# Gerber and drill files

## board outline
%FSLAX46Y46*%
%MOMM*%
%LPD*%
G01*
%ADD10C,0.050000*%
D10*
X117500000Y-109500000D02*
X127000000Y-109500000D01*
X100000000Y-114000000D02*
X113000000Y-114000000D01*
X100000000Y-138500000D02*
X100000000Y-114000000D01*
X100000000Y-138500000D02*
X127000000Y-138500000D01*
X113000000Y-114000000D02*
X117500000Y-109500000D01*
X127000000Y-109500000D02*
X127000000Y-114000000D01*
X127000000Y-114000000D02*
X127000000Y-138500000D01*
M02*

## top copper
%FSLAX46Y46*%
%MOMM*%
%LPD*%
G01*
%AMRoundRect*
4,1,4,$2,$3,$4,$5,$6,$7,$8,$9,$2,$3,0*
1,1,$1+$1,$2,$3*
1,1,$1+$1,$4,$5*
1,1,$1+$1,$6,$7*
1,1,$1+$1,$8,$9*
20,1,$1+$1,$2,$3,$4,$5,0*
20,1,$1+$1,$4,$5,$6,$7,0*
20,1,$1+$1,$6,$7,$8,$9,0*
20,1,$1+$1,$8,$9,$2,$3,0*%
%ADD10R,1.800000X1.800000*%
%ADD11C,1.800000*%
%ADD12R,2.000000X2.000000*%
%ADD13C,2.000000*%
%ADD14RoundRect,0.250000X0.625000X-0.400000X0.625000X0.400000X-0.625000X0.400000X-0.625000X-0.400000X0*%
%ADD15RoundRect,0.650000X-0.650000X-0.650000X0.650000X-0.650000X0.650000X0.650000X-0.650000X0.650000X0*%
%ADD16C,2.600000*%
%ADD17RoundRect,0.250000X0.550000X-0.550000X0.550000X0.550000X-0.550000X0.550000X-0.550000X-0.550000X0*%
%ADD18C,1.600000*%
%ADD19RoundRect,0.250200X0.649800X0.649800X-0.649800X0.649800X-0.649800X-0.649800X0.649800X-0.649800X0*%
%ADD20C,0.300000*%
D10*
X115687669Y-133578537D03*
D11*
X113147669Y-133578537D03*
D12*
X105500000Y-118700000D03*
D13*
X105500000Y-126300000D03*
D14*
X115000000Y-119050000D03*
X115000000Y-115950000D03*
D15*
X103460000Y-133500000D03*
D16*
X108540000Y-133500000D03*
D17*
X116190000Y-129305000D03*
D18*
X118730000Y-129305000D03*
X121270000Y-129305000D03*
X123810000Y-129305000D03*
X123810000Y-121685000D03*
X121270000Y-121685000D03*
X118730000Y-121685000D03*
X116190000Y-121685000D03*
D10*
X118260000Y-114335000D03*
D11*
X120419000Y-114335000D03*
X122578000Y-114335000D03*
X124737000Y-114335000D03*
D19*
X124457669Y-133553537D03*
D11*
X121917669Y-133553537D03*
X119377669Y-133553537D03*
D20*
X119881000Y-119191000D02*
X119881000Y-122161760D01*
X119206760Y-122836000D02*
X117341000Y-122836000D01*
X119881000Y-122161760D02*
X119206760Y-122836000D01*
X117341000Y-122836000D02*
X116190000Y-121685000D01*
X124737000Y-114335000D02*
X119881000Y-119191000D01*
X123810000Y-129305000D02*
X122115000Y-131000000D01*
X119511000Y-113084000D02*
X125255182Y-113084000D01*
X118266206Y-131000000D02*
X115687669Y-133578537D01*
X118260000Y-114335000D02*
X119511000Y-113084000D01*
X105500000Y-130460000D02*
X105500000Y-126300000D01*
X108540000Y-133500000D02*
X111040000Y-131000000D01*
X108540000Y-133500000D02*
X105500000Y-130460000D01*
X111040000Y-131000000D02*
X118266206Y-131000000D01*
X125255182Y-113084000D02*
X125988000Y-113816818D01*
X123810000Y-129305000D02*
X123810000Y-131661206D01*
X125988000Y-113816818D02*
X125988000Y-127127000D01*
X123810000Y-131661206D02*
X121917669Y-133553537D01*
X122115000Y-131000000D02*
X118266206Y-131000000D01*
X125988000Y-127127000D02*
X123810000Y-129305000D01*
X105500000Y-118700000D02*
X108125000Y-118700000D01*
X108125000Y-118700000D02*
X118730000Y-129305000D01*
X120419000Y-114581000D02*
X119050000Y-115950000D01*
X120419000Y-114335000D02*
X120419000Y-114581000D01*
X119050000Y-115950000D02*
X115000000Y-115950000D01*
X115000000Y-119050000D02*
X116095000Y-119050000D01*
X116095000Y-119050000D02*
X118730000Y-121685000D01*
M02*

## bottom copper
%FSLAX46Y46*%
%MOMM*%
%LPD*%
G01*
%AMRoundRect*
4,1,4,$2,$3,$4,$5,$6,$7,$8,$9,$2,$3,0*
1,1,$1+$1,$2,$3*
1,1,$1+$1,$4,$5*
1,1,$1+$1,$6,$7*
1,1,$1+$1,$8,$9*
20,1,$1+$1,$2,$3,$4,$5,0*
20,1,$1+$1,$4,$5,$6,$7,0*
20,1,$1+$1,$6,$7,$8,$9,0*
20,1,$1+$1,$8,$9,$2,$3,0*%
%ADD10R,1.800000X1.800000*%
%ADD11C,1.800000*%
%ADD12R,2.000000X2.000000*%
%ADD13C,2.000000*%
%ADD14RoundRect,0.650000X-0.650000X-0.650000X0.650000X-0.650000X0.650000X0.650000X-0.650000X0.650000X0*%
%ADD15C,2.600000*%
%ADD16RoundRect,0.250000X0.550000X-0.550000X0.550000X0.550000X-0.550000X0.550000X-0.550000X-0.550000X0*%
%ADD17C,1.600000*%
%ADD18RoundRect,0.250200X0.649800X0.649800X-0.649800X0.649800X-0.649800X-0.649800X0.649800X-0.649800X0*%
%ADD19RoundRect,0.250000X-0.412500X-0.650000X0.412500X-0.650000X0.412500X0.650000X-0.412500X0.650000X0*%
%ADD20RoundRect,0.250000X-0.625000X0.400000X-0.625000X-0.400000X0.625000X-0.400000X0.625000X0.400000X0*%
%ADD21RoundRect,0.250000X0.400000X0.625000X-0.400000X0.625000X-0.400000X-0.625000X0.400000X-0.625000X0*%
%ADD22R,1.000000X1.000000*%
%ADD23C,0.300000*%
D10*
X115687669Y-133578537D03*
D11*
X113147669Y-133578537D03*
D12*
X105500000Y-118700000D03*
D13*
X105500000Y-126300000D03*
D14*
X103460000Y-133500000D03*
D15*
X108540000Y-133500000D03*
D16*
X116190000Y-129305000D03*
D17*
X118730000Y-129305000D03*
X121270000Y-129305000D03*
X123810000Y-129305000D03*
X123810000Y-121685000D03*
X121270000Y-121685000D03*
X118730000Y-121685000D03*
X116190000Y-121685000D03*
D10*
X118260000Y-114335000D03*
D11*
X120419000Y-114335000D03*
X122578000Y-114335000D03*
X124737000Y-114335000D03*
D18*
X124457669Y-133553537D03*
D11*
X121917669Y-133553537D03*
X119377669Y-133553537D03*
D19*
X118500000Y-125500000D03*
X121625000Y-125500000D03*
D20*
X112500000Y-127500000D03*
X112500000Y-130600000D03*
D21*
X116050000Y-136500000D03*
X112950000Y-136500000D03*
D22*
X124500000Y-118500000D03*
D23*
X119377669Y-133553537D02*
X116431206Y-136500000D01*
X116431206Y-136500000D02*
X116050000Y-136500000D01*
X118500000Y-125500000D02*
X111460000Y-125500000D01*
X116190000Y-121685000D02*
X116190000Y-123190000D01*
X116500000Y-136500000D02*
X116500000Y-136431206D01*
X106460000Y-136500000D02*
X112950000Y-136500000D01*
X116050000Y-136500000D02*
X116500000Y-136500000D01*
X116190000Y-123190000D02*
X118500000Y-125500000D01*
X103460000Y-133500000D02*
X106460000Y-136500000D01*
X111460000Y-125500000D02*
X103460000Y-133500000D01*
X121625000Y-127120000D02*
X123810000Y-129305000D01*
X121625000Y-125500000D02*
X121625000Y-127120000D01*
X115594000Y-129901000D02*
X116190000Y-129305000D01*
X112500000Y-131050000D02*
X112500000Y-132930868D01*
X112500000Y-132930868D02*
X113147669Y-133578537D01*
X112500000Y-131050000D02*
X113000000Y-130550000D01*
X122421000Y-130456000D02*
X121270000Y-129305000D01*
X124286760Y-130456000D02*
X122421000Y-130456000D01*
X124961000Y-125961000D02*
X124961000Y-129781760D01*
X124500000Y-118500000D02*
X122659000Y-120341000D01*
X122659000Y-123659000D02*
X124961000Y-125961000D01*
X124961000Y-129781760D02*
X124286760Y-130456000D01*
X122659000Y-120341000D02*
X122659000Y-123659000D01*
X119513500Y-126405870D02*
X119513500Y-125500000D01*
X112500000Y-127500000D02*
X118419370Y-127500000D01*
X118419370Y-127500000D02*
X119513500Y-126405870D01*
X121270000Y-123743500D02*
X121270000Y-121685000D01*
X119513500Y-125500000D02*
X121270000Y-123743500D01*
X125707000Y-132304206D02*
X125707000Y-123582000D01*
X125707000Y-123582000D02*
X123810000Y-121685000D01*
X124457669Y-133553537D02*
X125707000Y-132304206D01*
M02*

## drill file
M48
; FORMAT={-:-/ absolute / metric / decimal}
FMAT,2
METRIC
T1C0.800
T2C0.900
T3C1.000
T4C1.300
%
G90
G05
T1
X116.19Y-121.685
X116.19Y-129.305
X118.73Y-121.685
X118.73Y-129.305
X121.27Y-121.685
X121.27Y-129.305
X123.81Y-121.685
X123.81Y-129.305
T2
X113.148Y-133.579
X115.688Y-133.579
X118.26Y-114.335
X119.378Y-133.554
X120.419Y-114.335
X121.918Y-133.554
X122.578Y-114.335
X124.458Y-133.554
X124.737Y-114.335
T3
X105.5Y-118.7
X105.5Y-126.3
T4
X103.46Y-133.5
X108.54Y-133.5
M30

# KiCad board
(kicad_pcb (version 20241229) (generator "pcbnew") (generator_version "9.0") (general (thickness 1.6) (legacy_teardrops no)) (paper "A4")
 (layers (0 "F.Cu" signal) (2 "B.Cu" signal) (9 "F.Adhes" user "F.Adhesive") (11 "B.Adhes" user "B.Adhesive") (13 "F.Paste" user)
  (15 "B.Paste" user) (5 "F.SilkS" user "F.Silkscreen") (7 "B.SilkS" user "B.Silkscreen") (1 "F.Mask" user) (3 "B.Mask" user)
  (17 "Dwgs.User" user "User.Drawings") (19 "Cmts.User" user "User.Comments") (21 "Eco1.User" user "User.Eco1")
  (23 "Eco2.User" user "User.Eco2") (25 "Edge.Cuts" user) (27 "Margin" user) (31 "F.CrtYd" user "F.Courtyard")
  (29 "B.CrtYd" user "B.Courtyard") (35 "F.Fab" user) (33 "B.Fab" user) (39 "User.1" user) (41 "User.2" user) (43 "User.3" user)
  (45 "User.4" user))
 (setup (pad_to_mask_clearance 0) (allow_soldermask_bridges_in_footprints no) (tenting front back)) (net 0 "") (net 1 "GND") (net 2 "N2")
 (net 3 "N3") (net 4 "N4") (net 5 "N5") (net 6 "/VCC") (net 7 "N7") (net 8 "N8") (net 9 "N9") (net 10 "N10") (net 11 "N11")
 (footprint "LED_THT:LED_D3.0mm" (layer "F.Cu") (at 115.687669 133.578537 180)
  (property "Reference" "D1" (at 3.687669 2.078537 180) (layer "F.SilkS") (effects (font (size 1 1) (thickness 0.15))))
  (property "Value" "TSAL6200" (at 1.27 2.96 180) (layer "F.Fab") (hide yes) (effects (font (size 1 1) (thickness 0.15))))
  (pad "1" thru_hole rect (at 0 0 180) (size 1.8 1.8) (drill 0.9) (layers "*.Cu" "*.Mask") (remove_unused_layers no) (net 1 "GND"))
  (pad "2" thru_hole circle (at 2.54 0 180) (size 1.8 1.8) (drill 0.9) (layers "*.Cu" "*.Mask") (remove_unused_layers no) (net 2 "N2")))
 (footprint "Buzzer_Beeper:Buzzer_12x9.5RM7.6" (layer "F.Cu") (at 105.5 118.7 -90)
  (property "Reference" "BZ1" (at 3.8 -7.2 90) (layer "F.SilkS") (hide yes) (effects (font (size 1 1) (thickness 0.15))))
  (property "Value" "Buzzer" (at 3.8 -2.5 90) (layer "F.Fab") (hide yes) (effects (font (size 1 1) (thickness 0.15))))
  (pad "1" thru_hole rect (at 0 0 270) (size 2 2) (drill 1) (layers "*.Cu" "*.Mask") (remove_unused_layers no) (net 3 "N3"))
  (pad "2" thru_hole circle (at 7.6 0 270) (size 2 2) (drill 1) (layers "*.Cu" "*.Mask") (remove_unused_layers no) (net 1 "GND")))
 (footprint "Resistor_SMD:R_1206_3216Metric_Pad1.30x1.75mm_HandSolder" (layer "F.Cu") (at 115 117.5 90)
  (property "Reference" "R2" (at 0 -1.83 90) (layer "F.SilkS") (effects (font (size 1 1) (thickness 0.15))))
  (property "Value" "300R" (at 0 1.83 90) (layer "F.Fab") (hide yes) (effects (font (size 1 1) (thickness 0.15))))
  (pad "1" smd roundrect (at -1.55 0 90) (size 1.3 1.75) (layers "F.Cu" "F.Mask" "F.Paste") (roundrect_rratio 0.192308) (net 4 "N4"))
  (pad "2" smd roundrect (at 1.55 0 90) (size 1.3 1.75) (layers "F.Cu" "F.Mask" "F.Paste") (roundrect_rratio 0.192308) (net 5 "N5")))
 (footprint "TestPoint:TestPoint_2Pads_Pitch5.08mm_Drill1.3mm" (layer "F.Cu") (at 103.46 133.5)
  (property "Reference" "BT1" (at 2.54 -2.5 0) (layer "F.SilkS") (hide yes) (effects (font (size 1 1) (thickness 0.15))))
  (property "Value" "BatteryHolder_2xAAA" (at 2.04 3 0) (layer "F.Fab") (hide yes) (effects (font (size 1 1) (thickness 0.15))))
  (pad "1" thru_hole roundrect (at 0 0) (size 2.6 2.6) (drill 1.3) (layers "*.Cu" "*.Mask") (remove_unused_layers no)
   (roundrect_rratio 0.25) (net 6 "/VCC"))
  (pad "2" thru_hole circle (at 5.08 0) (size 2.6 2.6) (drill 1.3) (layers "*.Cu" "*.Mask") (remove_unused_layers no) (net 1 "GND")))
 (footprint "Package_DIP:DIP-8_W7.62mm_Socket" (layer "F.Cu") (at 116.19 129.305 90)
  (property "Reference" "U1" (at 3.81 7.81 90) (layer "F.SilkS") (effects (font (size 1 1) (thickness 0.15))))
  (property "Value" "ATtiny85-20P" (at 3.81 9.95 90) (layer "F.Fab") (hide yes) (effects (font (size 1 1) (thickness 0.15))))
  (pad "1" thru_hole roundrect (at 0 0 90) (size 1.6 1.6) (drill 0.8) (layers "*.Cu" "*.Mask") (remove_unused_layers no)
   (roundrect_rratio 0.15625) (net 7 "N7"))
  (pad "2" thru_hole circle (at 0 2.54 90) (size 1.6 1.6) (drill 0.8) (layers "*.Cu" "*.Mask") (remove_unused_layers no) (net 3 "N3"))
  (pad "3" thru_hole circle (at 0 5.08 90) (size 1.6 1.6) (drill 0.8) (layers "*.Cu" "*.Mask") (remove_unused_layers no) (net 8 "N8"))
  (pad "4" thru_hole circle (at 0 7.62 90) (size 1.6 1.6) (drill 0.8) (layers "*.Cu" "*.Mask") (remove_unused_layers no) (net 1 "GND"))
  (pad "5" thru_hole circle (at 7.62 7.62 90) (size 1.6 1.6) (drill 0.8) (layers "*.Cu" "*.Mask") (remove_unused_layers no) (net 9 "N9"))
  (pad "6" thru_hole circle (at 7.62 5.08 90) (size 1.6 1.6) (drill 0.8) (layers "*.Cu" "*.Mask") (remove_unused_layers no) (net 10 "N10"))
  (pad "7" thru_hole circle (at 7.62 2.54 90) (size 1.6 1.6) (drill 0.8) (layers "*.Cu" "*.Mask") (remove_unused_layers no) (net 4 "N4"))
  (pad "8" thru_hole circle (at 7.62 0 90) (size 1.6 1.6) (drill 0.8) (layers "*.Cu" "*.Mask") (remove_unused_layers no) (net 6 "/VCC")))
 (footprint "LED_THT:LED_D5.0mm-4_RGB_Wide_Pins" (layer "F.Cu") (at 118.26 114.335)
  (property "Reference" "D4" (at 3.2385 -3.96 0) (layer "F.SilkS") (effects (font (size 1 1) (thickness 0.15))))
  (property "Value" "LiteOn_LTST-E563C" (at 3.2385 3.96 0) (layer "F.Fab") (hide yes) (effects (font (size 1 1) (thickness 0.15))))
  (pad "1" thru_hole rect (at 0 0) (size 1.8 1.8) (drill 0.9) (layers "*.Cu" "*.Mask") (remove_unused_layers no) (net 1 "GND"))
  (pad "2" thru_hole circle (at 2.159 0) (size 1.8 1.8) (drill 0.9) (layers "*.Cu" "*.Mask") (remove_unused_layers no) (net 5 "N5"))
  (pad "3" thru_hole circle (at 4.318 0) (size 1.8 1.8) (drill 0.9) (layers "*.Cu" "*.Mask") (remove_unused_layers no) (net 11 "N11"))
  (pad "4" thru_hole circle (at 6.477 0) (size 1.8 1.8) (drill 0.9) (layers "*.Cu" "*.Mask") (remove_unused_layers no) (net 6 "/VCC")))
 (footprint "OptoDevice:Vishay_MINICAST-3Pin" (layer "B.Cu") (at 124.457669 133.553537 180)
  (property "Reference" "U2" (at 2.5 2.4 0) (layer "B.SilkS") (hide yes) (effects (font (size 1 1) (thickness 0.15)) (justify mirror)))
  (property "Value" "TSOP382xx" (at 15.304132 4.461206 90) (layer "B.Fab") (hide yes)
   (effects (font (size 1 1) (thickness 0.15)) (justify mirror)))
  (pad "1" thru_hole roundrect (at 0 0 180) (size 1.8 1.8) (drill 0.9) (layers "*.Cu" "*.Mask") (remove_unused_layers no)
   (roundrect_rratio 0.139) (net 9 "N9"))
  (pad "2" thru_hole circle (at 2.54 0 180) (size 1.8 1.8) (drill 0.9) (layers "*.Cu" "*.Mask") (remove_unused_layers no) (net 1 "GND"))
  (pad "3" thru_hole circle (at 5.08 0 180) (size 1.8 1.8) (drill 0.9) (layers "*.Cu" "*.Mask") (remove_unused_layers no) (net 6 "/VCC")))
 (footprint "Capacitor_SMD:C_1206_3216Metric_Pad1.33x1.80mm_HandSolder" (layer "B.Cu") (at 120.0625 125.5)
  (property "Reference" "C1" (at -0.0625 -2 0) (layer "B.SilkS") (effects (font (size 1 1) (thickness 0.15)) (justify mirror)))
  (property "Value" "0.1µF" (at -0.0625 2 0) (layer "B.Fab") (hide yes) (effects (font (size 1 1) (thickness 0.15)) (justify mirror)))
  (pad "1" smd roundrect (at -1.5625 0) (size 1.325 1.8) (layers "B.Cu" "B.Mask" "B.Paste") (roundrect_rratio 0.188679) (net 6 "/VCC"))
  (pad "2" smd roundrect (at 1.5625 0) (size 1.325 1.8) (layers "B.Cu" "B.Mask" "B.Paste") (roundrect_rratio 0.188679) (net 1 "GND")))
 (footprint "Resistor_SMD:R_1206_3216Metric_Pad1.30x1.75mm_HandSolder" (layer "B.Cu") (at 112.5 129.05 -90)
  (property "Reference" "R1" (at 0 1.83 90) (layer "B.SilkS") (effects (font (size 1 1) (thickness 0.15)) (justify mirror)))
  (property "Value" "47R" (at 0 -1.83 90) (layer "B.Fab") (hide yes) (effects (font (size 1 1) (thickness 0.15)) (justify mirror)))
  (pad "1" smd roundrect (at -1.55 0 270) (size 1.3 1.75) (layers "B.Cu" "B.Mask" "B.Paste") (roundrect_rratio 0.192308) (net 10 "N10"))
  (pad "2" smd roundrect (at 1.55 0 270) (size 1.3 1.75) (layers "B.Cu" "B.Mask" "B.Paste") (roundrect_rratio 0.192308) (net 2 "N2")))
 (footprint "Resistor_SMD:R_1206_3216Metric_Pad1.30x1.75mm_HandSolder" (layer "B.Cu") (at 114.5 136.5 180)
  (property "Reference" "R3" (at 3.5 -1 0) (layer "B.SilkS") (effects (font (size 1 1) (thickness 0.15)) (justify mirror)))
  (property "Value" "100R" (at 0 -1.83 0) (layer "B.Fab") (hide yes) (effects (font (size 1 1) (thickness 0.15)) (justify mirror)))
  (pad "1" smd roundrect (at -1.55 0 180) (size 1.3 1.75) (layers "B.Cu" "B.Mask" "B.Paste") (roundrect_rratio 0.192308) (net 6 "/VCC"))
  (pad "2" smd roundrect (at 1.55 0 180) (size 1.3 1.75) (layers "B.Cu" "B.Mask" "B.Paste") (roundrect_rratio 0.192308) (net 6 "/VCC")))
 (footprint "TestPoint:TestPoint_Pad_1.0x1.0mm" (layer "B.Cu") (at 124.5 118.5 180)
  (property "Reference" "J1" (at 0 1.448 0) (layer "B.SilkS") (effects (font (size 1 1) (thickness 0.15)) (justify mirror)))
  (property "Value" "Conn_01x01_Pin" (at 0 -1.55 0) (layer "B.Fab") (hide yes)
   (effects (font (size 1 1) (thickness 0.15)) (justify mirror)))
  (pad "1" smd rect (at 0 0 180) (size 1 1) (layers "B.Cu" "B.Mask") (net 8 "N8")))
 (gr_line (start 117.5 109.5) (end 127 109.5) (stroke (width 0.05) (type default)) (layer "Edge.Cuts"))
 (gr_line (start 100 114) (end 113 114) (stroke (width 0.05) (type default)) (layer "Edge.Cuts"))
 (gr_line (start 100 138.5) (end 100 114) (stroke (width 0.05) (type default)) (layer "Edge.Cuts"))
 (gr_line (start 100 138.5) (end 127 138.5) (stroke (width 0.05) (type default)) (layer "Edge.Cuts"))
 (gr_line (start 113 114) (end 117.5 109.5) (stroke (width 0.05) (type default)) (layer "Edge.Cuts"))
 (gr_line (start 127 109.5) (end 127 114) (stroke (width 0.05) (type default)) (layer "Edge.Cuts"))
 (gr_line (start 127 114) (end 127 138.5) (stroke (width 0.05) (type default)) (layer "Edge.Cuts"))
 (segment (start 119.881 119.191) (end 119.881 122.16176) (width 0.3) (layer "F.Cu") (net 6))
 (segment (start 119.20676 122.836) (end 117.341 122.836) (width 0.3) (layer "F.Cu") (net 6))
 (segment (start 119.881 122.16176) (end 119.20676 122.836) (width 0.3) (layer "F.Cu") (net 6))
 (segment (start 117.341 122.836) (end 116.19 121.685) (width 0.3) (layer "F.Cu") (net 6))
 (segment (start 124.737 114.335) (end 119.881 119.191) (width 0.3) (layer "F.Cu") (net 6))
 (segment (start 119.377669 133.553537) (end 116.431206 136.5) (width 0.3) (layer "B.Cu") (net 6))
 (segment (start 116.431206 136.5) (end 116.05 136.5) (width 0.3) (layer "B.Cu") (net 6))
 (segment (start 118.5 125.5) (end 111.46 125.5) (width 0.3) (layer "B.Cu") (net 6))
 (segment (start 116.19 121.685) (end 116.19 123.19) (width 0.3) (layer "B.Cu") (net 6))
 (segment (start 116.5 136.5) (end 116.5 136.431206) (width 0.3) (layer "B.Cu") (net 6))
 (segment (start 106.46 136.5) (end 112.95 136.5) (width 0.3) (layer "B.Cu") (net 6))
 (segment (start 116.05 136.5) (end 116.5 136.5) (width 0.3) (layer "B.Cu") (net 6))
 (segment (start 116.19 123.19) (end 118.5 125.5) (width 0.3) (layer "B.Cu") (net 6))
 (segment (start 103.46 133.5) (end 106.46 136.5) (width 0.3) (layer "B.Cu") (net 6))
 (segment (start 111.46 125.5) (end 103.46 133.5) (width 0.3) (layer "B.Cu") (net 6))
 (segment (start 123.81 129.305) (end 122.115 131) (width 0.3) (layer "F.Cu") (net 1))
 (segment (start 119.511 113.084) (end 125.255182 113.084) (width 0.3) (layer "F.Cu") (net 1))
 (segment (start 118.266206 131) (end 115.687669 133.578537) (width 0.3) (layer "F.Cu") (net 1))
 (segment (start 118.26 114.335) (end 119.511 113.084) (width 0.3) (layer "F.Cu") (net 1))
 (segment (start 105.5 130.46) (end 105.5 126.3) (width 0.3) (layer "F.Cu") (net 1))
 (segment (start 108.54 133.5) (end 111.04 131) (width 0.3) (layer "F.Cu") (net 1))
 (segment (start 108.54 133.5) (end 105.5 130.46) (width 0.3) (layer "F.Cu") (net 1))
 (segment (start 111.04 131) (end 118.266206 131) (width 0.3) (layer "F.Cu") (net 1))
 (segment (start 125.255182 113.084) (end 125.988 113.816818) (width 0.3) (layer "F.Cu") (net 1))
 (segment (start 123.81 129.305) (end 123.81 131.661206) (width 0.3) (layer "F.Cu") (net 1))
 (segment (start 125.988 113.816818) (end 125.988 127.127) (width 0.3) (layer "F.Cu") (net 1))
 (segment (start 123.81 131.661206) (end 121.917669 133.553537) (width 0.3) (layer "F.Cu") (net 1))
 (segment (start 122.115 131) (end 118.266206 131) (width 0.3) (layer "F.Cu") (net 1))
 (segment (start 125.988 127.127) (end 123.81 129.305) (width 0.3) (layer "F.Cu") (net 1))
 (segment (start 121.625 127.12) (end 123.81 129.305) (width 0.3) (layer "B.Cu") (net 1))
 (segment (start 121.625 125.5) (end 121.625 127.12) (width 0.3) (layer "B.Cu") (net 1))
 (segment (start 115.594 129.901) (end 116.19 129.305) (width 0.3) (layer "B.Cu") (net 7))
 (segment (start 105.5 118.7) (end 108.125 118.7) (width 0.3) (layer "F.Cu") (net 3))
 (segment (start 108.125 118.7) (end 118.73 129.305) (width 0.3) (layer "F.Cu") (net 3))
 (segment (start 112.5 131.05) (end 112.5 132.930868) (width 0.3) (layer "B.Cu") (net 2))
 (segment (start 112.5 132.930868) (end 113.147669 133.578537) (width 0.3) (layer "B.Cu") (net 2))
 (segment (start 112.5 131.05) (end 113 130.55) (width 0.3) (layer "B.Cu") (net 2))
 (segment (start 120.419 114.581) (end 119.05 115.95) (width 0.3) (layer "F.Cu") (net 5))
 (segment (start 120.419 114.335) (end 120.419 114.581) (width 0.3) (layer "F.Cu") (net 5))
 (segment (start 119.05 115.95) (end 115 115.95) (width 0.3) (layer "F.Cu") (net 5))
 (segment (start 122.421 130.456) (end 121.27 129.305) (width 0.3) (layer "B.Cu") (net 8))
 (segment (start 124.28676 130.456) (end 122.421 130.456) (width 0.3) (layer "B.Cu") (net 8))
 (segment (start 124.961 125.961) (end 124.961 129.78176) (width 0.3) (layer "B.Cu") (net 8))
 (segment (start 124.5 118.5) (end 122.659 120.341) (width 0.3) (layer "B.Cu") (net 8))
 (segment (start 122.659 123.659) (end 124.961 125.961) (width 0.3) (layer "B.Cu") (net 8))
 (segment (start 124.961 129.78176) (end 124.28676 130.456) (width 0.3) (layer "B.Cu") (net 8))
 (segment (start 122.659 120.341) (end 122.659 123.659) (width 0.3) (layer "B.Cu") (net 8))
 (segment (start 119.5135 126.40587) (end 119.5135 125.5) (width 0.3) (layer "B.Cu") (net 10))
 (segment (start 112.5 127.5) (end 118.41937 127.5) (width 0.3) (layer "B.Cu") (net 10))
 (segment (start 118.41937 127.5) (end 119.5135 126.40587) (width 0.3) (layer "B.Cu") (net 10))
 (segment (start 121.27 123.7435) (end 121.27 121.685) (width 0.3) (layer "B.Cu") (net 10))
 (segment (start 119.5135 125.5) (end 121.27 123.7435) (width 0.3) (layer "B.Cu") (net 10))
 (segment (start 115 119.05) (end 116.095 119.05) (width 0.3) (layer "F.Cu") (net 4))
 (segment (start 116.095 119.05) (end 118.73 121.685) (width 0.3) (layer "F.Cu") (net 4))
 (segment (start 125.707 132.304206) (end 125.707 123.582) (width 0.3) (layer "B.Cu") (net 9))
 (segment (start 125.707 123.582) (end 123.81 121.685) (width 0.3) (layer "B.Cu") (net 9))
 (segment (start 124.457669 133.553537) (end 125.707 132.304206) (width 0.3) (layer "B.Cu") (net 9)))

